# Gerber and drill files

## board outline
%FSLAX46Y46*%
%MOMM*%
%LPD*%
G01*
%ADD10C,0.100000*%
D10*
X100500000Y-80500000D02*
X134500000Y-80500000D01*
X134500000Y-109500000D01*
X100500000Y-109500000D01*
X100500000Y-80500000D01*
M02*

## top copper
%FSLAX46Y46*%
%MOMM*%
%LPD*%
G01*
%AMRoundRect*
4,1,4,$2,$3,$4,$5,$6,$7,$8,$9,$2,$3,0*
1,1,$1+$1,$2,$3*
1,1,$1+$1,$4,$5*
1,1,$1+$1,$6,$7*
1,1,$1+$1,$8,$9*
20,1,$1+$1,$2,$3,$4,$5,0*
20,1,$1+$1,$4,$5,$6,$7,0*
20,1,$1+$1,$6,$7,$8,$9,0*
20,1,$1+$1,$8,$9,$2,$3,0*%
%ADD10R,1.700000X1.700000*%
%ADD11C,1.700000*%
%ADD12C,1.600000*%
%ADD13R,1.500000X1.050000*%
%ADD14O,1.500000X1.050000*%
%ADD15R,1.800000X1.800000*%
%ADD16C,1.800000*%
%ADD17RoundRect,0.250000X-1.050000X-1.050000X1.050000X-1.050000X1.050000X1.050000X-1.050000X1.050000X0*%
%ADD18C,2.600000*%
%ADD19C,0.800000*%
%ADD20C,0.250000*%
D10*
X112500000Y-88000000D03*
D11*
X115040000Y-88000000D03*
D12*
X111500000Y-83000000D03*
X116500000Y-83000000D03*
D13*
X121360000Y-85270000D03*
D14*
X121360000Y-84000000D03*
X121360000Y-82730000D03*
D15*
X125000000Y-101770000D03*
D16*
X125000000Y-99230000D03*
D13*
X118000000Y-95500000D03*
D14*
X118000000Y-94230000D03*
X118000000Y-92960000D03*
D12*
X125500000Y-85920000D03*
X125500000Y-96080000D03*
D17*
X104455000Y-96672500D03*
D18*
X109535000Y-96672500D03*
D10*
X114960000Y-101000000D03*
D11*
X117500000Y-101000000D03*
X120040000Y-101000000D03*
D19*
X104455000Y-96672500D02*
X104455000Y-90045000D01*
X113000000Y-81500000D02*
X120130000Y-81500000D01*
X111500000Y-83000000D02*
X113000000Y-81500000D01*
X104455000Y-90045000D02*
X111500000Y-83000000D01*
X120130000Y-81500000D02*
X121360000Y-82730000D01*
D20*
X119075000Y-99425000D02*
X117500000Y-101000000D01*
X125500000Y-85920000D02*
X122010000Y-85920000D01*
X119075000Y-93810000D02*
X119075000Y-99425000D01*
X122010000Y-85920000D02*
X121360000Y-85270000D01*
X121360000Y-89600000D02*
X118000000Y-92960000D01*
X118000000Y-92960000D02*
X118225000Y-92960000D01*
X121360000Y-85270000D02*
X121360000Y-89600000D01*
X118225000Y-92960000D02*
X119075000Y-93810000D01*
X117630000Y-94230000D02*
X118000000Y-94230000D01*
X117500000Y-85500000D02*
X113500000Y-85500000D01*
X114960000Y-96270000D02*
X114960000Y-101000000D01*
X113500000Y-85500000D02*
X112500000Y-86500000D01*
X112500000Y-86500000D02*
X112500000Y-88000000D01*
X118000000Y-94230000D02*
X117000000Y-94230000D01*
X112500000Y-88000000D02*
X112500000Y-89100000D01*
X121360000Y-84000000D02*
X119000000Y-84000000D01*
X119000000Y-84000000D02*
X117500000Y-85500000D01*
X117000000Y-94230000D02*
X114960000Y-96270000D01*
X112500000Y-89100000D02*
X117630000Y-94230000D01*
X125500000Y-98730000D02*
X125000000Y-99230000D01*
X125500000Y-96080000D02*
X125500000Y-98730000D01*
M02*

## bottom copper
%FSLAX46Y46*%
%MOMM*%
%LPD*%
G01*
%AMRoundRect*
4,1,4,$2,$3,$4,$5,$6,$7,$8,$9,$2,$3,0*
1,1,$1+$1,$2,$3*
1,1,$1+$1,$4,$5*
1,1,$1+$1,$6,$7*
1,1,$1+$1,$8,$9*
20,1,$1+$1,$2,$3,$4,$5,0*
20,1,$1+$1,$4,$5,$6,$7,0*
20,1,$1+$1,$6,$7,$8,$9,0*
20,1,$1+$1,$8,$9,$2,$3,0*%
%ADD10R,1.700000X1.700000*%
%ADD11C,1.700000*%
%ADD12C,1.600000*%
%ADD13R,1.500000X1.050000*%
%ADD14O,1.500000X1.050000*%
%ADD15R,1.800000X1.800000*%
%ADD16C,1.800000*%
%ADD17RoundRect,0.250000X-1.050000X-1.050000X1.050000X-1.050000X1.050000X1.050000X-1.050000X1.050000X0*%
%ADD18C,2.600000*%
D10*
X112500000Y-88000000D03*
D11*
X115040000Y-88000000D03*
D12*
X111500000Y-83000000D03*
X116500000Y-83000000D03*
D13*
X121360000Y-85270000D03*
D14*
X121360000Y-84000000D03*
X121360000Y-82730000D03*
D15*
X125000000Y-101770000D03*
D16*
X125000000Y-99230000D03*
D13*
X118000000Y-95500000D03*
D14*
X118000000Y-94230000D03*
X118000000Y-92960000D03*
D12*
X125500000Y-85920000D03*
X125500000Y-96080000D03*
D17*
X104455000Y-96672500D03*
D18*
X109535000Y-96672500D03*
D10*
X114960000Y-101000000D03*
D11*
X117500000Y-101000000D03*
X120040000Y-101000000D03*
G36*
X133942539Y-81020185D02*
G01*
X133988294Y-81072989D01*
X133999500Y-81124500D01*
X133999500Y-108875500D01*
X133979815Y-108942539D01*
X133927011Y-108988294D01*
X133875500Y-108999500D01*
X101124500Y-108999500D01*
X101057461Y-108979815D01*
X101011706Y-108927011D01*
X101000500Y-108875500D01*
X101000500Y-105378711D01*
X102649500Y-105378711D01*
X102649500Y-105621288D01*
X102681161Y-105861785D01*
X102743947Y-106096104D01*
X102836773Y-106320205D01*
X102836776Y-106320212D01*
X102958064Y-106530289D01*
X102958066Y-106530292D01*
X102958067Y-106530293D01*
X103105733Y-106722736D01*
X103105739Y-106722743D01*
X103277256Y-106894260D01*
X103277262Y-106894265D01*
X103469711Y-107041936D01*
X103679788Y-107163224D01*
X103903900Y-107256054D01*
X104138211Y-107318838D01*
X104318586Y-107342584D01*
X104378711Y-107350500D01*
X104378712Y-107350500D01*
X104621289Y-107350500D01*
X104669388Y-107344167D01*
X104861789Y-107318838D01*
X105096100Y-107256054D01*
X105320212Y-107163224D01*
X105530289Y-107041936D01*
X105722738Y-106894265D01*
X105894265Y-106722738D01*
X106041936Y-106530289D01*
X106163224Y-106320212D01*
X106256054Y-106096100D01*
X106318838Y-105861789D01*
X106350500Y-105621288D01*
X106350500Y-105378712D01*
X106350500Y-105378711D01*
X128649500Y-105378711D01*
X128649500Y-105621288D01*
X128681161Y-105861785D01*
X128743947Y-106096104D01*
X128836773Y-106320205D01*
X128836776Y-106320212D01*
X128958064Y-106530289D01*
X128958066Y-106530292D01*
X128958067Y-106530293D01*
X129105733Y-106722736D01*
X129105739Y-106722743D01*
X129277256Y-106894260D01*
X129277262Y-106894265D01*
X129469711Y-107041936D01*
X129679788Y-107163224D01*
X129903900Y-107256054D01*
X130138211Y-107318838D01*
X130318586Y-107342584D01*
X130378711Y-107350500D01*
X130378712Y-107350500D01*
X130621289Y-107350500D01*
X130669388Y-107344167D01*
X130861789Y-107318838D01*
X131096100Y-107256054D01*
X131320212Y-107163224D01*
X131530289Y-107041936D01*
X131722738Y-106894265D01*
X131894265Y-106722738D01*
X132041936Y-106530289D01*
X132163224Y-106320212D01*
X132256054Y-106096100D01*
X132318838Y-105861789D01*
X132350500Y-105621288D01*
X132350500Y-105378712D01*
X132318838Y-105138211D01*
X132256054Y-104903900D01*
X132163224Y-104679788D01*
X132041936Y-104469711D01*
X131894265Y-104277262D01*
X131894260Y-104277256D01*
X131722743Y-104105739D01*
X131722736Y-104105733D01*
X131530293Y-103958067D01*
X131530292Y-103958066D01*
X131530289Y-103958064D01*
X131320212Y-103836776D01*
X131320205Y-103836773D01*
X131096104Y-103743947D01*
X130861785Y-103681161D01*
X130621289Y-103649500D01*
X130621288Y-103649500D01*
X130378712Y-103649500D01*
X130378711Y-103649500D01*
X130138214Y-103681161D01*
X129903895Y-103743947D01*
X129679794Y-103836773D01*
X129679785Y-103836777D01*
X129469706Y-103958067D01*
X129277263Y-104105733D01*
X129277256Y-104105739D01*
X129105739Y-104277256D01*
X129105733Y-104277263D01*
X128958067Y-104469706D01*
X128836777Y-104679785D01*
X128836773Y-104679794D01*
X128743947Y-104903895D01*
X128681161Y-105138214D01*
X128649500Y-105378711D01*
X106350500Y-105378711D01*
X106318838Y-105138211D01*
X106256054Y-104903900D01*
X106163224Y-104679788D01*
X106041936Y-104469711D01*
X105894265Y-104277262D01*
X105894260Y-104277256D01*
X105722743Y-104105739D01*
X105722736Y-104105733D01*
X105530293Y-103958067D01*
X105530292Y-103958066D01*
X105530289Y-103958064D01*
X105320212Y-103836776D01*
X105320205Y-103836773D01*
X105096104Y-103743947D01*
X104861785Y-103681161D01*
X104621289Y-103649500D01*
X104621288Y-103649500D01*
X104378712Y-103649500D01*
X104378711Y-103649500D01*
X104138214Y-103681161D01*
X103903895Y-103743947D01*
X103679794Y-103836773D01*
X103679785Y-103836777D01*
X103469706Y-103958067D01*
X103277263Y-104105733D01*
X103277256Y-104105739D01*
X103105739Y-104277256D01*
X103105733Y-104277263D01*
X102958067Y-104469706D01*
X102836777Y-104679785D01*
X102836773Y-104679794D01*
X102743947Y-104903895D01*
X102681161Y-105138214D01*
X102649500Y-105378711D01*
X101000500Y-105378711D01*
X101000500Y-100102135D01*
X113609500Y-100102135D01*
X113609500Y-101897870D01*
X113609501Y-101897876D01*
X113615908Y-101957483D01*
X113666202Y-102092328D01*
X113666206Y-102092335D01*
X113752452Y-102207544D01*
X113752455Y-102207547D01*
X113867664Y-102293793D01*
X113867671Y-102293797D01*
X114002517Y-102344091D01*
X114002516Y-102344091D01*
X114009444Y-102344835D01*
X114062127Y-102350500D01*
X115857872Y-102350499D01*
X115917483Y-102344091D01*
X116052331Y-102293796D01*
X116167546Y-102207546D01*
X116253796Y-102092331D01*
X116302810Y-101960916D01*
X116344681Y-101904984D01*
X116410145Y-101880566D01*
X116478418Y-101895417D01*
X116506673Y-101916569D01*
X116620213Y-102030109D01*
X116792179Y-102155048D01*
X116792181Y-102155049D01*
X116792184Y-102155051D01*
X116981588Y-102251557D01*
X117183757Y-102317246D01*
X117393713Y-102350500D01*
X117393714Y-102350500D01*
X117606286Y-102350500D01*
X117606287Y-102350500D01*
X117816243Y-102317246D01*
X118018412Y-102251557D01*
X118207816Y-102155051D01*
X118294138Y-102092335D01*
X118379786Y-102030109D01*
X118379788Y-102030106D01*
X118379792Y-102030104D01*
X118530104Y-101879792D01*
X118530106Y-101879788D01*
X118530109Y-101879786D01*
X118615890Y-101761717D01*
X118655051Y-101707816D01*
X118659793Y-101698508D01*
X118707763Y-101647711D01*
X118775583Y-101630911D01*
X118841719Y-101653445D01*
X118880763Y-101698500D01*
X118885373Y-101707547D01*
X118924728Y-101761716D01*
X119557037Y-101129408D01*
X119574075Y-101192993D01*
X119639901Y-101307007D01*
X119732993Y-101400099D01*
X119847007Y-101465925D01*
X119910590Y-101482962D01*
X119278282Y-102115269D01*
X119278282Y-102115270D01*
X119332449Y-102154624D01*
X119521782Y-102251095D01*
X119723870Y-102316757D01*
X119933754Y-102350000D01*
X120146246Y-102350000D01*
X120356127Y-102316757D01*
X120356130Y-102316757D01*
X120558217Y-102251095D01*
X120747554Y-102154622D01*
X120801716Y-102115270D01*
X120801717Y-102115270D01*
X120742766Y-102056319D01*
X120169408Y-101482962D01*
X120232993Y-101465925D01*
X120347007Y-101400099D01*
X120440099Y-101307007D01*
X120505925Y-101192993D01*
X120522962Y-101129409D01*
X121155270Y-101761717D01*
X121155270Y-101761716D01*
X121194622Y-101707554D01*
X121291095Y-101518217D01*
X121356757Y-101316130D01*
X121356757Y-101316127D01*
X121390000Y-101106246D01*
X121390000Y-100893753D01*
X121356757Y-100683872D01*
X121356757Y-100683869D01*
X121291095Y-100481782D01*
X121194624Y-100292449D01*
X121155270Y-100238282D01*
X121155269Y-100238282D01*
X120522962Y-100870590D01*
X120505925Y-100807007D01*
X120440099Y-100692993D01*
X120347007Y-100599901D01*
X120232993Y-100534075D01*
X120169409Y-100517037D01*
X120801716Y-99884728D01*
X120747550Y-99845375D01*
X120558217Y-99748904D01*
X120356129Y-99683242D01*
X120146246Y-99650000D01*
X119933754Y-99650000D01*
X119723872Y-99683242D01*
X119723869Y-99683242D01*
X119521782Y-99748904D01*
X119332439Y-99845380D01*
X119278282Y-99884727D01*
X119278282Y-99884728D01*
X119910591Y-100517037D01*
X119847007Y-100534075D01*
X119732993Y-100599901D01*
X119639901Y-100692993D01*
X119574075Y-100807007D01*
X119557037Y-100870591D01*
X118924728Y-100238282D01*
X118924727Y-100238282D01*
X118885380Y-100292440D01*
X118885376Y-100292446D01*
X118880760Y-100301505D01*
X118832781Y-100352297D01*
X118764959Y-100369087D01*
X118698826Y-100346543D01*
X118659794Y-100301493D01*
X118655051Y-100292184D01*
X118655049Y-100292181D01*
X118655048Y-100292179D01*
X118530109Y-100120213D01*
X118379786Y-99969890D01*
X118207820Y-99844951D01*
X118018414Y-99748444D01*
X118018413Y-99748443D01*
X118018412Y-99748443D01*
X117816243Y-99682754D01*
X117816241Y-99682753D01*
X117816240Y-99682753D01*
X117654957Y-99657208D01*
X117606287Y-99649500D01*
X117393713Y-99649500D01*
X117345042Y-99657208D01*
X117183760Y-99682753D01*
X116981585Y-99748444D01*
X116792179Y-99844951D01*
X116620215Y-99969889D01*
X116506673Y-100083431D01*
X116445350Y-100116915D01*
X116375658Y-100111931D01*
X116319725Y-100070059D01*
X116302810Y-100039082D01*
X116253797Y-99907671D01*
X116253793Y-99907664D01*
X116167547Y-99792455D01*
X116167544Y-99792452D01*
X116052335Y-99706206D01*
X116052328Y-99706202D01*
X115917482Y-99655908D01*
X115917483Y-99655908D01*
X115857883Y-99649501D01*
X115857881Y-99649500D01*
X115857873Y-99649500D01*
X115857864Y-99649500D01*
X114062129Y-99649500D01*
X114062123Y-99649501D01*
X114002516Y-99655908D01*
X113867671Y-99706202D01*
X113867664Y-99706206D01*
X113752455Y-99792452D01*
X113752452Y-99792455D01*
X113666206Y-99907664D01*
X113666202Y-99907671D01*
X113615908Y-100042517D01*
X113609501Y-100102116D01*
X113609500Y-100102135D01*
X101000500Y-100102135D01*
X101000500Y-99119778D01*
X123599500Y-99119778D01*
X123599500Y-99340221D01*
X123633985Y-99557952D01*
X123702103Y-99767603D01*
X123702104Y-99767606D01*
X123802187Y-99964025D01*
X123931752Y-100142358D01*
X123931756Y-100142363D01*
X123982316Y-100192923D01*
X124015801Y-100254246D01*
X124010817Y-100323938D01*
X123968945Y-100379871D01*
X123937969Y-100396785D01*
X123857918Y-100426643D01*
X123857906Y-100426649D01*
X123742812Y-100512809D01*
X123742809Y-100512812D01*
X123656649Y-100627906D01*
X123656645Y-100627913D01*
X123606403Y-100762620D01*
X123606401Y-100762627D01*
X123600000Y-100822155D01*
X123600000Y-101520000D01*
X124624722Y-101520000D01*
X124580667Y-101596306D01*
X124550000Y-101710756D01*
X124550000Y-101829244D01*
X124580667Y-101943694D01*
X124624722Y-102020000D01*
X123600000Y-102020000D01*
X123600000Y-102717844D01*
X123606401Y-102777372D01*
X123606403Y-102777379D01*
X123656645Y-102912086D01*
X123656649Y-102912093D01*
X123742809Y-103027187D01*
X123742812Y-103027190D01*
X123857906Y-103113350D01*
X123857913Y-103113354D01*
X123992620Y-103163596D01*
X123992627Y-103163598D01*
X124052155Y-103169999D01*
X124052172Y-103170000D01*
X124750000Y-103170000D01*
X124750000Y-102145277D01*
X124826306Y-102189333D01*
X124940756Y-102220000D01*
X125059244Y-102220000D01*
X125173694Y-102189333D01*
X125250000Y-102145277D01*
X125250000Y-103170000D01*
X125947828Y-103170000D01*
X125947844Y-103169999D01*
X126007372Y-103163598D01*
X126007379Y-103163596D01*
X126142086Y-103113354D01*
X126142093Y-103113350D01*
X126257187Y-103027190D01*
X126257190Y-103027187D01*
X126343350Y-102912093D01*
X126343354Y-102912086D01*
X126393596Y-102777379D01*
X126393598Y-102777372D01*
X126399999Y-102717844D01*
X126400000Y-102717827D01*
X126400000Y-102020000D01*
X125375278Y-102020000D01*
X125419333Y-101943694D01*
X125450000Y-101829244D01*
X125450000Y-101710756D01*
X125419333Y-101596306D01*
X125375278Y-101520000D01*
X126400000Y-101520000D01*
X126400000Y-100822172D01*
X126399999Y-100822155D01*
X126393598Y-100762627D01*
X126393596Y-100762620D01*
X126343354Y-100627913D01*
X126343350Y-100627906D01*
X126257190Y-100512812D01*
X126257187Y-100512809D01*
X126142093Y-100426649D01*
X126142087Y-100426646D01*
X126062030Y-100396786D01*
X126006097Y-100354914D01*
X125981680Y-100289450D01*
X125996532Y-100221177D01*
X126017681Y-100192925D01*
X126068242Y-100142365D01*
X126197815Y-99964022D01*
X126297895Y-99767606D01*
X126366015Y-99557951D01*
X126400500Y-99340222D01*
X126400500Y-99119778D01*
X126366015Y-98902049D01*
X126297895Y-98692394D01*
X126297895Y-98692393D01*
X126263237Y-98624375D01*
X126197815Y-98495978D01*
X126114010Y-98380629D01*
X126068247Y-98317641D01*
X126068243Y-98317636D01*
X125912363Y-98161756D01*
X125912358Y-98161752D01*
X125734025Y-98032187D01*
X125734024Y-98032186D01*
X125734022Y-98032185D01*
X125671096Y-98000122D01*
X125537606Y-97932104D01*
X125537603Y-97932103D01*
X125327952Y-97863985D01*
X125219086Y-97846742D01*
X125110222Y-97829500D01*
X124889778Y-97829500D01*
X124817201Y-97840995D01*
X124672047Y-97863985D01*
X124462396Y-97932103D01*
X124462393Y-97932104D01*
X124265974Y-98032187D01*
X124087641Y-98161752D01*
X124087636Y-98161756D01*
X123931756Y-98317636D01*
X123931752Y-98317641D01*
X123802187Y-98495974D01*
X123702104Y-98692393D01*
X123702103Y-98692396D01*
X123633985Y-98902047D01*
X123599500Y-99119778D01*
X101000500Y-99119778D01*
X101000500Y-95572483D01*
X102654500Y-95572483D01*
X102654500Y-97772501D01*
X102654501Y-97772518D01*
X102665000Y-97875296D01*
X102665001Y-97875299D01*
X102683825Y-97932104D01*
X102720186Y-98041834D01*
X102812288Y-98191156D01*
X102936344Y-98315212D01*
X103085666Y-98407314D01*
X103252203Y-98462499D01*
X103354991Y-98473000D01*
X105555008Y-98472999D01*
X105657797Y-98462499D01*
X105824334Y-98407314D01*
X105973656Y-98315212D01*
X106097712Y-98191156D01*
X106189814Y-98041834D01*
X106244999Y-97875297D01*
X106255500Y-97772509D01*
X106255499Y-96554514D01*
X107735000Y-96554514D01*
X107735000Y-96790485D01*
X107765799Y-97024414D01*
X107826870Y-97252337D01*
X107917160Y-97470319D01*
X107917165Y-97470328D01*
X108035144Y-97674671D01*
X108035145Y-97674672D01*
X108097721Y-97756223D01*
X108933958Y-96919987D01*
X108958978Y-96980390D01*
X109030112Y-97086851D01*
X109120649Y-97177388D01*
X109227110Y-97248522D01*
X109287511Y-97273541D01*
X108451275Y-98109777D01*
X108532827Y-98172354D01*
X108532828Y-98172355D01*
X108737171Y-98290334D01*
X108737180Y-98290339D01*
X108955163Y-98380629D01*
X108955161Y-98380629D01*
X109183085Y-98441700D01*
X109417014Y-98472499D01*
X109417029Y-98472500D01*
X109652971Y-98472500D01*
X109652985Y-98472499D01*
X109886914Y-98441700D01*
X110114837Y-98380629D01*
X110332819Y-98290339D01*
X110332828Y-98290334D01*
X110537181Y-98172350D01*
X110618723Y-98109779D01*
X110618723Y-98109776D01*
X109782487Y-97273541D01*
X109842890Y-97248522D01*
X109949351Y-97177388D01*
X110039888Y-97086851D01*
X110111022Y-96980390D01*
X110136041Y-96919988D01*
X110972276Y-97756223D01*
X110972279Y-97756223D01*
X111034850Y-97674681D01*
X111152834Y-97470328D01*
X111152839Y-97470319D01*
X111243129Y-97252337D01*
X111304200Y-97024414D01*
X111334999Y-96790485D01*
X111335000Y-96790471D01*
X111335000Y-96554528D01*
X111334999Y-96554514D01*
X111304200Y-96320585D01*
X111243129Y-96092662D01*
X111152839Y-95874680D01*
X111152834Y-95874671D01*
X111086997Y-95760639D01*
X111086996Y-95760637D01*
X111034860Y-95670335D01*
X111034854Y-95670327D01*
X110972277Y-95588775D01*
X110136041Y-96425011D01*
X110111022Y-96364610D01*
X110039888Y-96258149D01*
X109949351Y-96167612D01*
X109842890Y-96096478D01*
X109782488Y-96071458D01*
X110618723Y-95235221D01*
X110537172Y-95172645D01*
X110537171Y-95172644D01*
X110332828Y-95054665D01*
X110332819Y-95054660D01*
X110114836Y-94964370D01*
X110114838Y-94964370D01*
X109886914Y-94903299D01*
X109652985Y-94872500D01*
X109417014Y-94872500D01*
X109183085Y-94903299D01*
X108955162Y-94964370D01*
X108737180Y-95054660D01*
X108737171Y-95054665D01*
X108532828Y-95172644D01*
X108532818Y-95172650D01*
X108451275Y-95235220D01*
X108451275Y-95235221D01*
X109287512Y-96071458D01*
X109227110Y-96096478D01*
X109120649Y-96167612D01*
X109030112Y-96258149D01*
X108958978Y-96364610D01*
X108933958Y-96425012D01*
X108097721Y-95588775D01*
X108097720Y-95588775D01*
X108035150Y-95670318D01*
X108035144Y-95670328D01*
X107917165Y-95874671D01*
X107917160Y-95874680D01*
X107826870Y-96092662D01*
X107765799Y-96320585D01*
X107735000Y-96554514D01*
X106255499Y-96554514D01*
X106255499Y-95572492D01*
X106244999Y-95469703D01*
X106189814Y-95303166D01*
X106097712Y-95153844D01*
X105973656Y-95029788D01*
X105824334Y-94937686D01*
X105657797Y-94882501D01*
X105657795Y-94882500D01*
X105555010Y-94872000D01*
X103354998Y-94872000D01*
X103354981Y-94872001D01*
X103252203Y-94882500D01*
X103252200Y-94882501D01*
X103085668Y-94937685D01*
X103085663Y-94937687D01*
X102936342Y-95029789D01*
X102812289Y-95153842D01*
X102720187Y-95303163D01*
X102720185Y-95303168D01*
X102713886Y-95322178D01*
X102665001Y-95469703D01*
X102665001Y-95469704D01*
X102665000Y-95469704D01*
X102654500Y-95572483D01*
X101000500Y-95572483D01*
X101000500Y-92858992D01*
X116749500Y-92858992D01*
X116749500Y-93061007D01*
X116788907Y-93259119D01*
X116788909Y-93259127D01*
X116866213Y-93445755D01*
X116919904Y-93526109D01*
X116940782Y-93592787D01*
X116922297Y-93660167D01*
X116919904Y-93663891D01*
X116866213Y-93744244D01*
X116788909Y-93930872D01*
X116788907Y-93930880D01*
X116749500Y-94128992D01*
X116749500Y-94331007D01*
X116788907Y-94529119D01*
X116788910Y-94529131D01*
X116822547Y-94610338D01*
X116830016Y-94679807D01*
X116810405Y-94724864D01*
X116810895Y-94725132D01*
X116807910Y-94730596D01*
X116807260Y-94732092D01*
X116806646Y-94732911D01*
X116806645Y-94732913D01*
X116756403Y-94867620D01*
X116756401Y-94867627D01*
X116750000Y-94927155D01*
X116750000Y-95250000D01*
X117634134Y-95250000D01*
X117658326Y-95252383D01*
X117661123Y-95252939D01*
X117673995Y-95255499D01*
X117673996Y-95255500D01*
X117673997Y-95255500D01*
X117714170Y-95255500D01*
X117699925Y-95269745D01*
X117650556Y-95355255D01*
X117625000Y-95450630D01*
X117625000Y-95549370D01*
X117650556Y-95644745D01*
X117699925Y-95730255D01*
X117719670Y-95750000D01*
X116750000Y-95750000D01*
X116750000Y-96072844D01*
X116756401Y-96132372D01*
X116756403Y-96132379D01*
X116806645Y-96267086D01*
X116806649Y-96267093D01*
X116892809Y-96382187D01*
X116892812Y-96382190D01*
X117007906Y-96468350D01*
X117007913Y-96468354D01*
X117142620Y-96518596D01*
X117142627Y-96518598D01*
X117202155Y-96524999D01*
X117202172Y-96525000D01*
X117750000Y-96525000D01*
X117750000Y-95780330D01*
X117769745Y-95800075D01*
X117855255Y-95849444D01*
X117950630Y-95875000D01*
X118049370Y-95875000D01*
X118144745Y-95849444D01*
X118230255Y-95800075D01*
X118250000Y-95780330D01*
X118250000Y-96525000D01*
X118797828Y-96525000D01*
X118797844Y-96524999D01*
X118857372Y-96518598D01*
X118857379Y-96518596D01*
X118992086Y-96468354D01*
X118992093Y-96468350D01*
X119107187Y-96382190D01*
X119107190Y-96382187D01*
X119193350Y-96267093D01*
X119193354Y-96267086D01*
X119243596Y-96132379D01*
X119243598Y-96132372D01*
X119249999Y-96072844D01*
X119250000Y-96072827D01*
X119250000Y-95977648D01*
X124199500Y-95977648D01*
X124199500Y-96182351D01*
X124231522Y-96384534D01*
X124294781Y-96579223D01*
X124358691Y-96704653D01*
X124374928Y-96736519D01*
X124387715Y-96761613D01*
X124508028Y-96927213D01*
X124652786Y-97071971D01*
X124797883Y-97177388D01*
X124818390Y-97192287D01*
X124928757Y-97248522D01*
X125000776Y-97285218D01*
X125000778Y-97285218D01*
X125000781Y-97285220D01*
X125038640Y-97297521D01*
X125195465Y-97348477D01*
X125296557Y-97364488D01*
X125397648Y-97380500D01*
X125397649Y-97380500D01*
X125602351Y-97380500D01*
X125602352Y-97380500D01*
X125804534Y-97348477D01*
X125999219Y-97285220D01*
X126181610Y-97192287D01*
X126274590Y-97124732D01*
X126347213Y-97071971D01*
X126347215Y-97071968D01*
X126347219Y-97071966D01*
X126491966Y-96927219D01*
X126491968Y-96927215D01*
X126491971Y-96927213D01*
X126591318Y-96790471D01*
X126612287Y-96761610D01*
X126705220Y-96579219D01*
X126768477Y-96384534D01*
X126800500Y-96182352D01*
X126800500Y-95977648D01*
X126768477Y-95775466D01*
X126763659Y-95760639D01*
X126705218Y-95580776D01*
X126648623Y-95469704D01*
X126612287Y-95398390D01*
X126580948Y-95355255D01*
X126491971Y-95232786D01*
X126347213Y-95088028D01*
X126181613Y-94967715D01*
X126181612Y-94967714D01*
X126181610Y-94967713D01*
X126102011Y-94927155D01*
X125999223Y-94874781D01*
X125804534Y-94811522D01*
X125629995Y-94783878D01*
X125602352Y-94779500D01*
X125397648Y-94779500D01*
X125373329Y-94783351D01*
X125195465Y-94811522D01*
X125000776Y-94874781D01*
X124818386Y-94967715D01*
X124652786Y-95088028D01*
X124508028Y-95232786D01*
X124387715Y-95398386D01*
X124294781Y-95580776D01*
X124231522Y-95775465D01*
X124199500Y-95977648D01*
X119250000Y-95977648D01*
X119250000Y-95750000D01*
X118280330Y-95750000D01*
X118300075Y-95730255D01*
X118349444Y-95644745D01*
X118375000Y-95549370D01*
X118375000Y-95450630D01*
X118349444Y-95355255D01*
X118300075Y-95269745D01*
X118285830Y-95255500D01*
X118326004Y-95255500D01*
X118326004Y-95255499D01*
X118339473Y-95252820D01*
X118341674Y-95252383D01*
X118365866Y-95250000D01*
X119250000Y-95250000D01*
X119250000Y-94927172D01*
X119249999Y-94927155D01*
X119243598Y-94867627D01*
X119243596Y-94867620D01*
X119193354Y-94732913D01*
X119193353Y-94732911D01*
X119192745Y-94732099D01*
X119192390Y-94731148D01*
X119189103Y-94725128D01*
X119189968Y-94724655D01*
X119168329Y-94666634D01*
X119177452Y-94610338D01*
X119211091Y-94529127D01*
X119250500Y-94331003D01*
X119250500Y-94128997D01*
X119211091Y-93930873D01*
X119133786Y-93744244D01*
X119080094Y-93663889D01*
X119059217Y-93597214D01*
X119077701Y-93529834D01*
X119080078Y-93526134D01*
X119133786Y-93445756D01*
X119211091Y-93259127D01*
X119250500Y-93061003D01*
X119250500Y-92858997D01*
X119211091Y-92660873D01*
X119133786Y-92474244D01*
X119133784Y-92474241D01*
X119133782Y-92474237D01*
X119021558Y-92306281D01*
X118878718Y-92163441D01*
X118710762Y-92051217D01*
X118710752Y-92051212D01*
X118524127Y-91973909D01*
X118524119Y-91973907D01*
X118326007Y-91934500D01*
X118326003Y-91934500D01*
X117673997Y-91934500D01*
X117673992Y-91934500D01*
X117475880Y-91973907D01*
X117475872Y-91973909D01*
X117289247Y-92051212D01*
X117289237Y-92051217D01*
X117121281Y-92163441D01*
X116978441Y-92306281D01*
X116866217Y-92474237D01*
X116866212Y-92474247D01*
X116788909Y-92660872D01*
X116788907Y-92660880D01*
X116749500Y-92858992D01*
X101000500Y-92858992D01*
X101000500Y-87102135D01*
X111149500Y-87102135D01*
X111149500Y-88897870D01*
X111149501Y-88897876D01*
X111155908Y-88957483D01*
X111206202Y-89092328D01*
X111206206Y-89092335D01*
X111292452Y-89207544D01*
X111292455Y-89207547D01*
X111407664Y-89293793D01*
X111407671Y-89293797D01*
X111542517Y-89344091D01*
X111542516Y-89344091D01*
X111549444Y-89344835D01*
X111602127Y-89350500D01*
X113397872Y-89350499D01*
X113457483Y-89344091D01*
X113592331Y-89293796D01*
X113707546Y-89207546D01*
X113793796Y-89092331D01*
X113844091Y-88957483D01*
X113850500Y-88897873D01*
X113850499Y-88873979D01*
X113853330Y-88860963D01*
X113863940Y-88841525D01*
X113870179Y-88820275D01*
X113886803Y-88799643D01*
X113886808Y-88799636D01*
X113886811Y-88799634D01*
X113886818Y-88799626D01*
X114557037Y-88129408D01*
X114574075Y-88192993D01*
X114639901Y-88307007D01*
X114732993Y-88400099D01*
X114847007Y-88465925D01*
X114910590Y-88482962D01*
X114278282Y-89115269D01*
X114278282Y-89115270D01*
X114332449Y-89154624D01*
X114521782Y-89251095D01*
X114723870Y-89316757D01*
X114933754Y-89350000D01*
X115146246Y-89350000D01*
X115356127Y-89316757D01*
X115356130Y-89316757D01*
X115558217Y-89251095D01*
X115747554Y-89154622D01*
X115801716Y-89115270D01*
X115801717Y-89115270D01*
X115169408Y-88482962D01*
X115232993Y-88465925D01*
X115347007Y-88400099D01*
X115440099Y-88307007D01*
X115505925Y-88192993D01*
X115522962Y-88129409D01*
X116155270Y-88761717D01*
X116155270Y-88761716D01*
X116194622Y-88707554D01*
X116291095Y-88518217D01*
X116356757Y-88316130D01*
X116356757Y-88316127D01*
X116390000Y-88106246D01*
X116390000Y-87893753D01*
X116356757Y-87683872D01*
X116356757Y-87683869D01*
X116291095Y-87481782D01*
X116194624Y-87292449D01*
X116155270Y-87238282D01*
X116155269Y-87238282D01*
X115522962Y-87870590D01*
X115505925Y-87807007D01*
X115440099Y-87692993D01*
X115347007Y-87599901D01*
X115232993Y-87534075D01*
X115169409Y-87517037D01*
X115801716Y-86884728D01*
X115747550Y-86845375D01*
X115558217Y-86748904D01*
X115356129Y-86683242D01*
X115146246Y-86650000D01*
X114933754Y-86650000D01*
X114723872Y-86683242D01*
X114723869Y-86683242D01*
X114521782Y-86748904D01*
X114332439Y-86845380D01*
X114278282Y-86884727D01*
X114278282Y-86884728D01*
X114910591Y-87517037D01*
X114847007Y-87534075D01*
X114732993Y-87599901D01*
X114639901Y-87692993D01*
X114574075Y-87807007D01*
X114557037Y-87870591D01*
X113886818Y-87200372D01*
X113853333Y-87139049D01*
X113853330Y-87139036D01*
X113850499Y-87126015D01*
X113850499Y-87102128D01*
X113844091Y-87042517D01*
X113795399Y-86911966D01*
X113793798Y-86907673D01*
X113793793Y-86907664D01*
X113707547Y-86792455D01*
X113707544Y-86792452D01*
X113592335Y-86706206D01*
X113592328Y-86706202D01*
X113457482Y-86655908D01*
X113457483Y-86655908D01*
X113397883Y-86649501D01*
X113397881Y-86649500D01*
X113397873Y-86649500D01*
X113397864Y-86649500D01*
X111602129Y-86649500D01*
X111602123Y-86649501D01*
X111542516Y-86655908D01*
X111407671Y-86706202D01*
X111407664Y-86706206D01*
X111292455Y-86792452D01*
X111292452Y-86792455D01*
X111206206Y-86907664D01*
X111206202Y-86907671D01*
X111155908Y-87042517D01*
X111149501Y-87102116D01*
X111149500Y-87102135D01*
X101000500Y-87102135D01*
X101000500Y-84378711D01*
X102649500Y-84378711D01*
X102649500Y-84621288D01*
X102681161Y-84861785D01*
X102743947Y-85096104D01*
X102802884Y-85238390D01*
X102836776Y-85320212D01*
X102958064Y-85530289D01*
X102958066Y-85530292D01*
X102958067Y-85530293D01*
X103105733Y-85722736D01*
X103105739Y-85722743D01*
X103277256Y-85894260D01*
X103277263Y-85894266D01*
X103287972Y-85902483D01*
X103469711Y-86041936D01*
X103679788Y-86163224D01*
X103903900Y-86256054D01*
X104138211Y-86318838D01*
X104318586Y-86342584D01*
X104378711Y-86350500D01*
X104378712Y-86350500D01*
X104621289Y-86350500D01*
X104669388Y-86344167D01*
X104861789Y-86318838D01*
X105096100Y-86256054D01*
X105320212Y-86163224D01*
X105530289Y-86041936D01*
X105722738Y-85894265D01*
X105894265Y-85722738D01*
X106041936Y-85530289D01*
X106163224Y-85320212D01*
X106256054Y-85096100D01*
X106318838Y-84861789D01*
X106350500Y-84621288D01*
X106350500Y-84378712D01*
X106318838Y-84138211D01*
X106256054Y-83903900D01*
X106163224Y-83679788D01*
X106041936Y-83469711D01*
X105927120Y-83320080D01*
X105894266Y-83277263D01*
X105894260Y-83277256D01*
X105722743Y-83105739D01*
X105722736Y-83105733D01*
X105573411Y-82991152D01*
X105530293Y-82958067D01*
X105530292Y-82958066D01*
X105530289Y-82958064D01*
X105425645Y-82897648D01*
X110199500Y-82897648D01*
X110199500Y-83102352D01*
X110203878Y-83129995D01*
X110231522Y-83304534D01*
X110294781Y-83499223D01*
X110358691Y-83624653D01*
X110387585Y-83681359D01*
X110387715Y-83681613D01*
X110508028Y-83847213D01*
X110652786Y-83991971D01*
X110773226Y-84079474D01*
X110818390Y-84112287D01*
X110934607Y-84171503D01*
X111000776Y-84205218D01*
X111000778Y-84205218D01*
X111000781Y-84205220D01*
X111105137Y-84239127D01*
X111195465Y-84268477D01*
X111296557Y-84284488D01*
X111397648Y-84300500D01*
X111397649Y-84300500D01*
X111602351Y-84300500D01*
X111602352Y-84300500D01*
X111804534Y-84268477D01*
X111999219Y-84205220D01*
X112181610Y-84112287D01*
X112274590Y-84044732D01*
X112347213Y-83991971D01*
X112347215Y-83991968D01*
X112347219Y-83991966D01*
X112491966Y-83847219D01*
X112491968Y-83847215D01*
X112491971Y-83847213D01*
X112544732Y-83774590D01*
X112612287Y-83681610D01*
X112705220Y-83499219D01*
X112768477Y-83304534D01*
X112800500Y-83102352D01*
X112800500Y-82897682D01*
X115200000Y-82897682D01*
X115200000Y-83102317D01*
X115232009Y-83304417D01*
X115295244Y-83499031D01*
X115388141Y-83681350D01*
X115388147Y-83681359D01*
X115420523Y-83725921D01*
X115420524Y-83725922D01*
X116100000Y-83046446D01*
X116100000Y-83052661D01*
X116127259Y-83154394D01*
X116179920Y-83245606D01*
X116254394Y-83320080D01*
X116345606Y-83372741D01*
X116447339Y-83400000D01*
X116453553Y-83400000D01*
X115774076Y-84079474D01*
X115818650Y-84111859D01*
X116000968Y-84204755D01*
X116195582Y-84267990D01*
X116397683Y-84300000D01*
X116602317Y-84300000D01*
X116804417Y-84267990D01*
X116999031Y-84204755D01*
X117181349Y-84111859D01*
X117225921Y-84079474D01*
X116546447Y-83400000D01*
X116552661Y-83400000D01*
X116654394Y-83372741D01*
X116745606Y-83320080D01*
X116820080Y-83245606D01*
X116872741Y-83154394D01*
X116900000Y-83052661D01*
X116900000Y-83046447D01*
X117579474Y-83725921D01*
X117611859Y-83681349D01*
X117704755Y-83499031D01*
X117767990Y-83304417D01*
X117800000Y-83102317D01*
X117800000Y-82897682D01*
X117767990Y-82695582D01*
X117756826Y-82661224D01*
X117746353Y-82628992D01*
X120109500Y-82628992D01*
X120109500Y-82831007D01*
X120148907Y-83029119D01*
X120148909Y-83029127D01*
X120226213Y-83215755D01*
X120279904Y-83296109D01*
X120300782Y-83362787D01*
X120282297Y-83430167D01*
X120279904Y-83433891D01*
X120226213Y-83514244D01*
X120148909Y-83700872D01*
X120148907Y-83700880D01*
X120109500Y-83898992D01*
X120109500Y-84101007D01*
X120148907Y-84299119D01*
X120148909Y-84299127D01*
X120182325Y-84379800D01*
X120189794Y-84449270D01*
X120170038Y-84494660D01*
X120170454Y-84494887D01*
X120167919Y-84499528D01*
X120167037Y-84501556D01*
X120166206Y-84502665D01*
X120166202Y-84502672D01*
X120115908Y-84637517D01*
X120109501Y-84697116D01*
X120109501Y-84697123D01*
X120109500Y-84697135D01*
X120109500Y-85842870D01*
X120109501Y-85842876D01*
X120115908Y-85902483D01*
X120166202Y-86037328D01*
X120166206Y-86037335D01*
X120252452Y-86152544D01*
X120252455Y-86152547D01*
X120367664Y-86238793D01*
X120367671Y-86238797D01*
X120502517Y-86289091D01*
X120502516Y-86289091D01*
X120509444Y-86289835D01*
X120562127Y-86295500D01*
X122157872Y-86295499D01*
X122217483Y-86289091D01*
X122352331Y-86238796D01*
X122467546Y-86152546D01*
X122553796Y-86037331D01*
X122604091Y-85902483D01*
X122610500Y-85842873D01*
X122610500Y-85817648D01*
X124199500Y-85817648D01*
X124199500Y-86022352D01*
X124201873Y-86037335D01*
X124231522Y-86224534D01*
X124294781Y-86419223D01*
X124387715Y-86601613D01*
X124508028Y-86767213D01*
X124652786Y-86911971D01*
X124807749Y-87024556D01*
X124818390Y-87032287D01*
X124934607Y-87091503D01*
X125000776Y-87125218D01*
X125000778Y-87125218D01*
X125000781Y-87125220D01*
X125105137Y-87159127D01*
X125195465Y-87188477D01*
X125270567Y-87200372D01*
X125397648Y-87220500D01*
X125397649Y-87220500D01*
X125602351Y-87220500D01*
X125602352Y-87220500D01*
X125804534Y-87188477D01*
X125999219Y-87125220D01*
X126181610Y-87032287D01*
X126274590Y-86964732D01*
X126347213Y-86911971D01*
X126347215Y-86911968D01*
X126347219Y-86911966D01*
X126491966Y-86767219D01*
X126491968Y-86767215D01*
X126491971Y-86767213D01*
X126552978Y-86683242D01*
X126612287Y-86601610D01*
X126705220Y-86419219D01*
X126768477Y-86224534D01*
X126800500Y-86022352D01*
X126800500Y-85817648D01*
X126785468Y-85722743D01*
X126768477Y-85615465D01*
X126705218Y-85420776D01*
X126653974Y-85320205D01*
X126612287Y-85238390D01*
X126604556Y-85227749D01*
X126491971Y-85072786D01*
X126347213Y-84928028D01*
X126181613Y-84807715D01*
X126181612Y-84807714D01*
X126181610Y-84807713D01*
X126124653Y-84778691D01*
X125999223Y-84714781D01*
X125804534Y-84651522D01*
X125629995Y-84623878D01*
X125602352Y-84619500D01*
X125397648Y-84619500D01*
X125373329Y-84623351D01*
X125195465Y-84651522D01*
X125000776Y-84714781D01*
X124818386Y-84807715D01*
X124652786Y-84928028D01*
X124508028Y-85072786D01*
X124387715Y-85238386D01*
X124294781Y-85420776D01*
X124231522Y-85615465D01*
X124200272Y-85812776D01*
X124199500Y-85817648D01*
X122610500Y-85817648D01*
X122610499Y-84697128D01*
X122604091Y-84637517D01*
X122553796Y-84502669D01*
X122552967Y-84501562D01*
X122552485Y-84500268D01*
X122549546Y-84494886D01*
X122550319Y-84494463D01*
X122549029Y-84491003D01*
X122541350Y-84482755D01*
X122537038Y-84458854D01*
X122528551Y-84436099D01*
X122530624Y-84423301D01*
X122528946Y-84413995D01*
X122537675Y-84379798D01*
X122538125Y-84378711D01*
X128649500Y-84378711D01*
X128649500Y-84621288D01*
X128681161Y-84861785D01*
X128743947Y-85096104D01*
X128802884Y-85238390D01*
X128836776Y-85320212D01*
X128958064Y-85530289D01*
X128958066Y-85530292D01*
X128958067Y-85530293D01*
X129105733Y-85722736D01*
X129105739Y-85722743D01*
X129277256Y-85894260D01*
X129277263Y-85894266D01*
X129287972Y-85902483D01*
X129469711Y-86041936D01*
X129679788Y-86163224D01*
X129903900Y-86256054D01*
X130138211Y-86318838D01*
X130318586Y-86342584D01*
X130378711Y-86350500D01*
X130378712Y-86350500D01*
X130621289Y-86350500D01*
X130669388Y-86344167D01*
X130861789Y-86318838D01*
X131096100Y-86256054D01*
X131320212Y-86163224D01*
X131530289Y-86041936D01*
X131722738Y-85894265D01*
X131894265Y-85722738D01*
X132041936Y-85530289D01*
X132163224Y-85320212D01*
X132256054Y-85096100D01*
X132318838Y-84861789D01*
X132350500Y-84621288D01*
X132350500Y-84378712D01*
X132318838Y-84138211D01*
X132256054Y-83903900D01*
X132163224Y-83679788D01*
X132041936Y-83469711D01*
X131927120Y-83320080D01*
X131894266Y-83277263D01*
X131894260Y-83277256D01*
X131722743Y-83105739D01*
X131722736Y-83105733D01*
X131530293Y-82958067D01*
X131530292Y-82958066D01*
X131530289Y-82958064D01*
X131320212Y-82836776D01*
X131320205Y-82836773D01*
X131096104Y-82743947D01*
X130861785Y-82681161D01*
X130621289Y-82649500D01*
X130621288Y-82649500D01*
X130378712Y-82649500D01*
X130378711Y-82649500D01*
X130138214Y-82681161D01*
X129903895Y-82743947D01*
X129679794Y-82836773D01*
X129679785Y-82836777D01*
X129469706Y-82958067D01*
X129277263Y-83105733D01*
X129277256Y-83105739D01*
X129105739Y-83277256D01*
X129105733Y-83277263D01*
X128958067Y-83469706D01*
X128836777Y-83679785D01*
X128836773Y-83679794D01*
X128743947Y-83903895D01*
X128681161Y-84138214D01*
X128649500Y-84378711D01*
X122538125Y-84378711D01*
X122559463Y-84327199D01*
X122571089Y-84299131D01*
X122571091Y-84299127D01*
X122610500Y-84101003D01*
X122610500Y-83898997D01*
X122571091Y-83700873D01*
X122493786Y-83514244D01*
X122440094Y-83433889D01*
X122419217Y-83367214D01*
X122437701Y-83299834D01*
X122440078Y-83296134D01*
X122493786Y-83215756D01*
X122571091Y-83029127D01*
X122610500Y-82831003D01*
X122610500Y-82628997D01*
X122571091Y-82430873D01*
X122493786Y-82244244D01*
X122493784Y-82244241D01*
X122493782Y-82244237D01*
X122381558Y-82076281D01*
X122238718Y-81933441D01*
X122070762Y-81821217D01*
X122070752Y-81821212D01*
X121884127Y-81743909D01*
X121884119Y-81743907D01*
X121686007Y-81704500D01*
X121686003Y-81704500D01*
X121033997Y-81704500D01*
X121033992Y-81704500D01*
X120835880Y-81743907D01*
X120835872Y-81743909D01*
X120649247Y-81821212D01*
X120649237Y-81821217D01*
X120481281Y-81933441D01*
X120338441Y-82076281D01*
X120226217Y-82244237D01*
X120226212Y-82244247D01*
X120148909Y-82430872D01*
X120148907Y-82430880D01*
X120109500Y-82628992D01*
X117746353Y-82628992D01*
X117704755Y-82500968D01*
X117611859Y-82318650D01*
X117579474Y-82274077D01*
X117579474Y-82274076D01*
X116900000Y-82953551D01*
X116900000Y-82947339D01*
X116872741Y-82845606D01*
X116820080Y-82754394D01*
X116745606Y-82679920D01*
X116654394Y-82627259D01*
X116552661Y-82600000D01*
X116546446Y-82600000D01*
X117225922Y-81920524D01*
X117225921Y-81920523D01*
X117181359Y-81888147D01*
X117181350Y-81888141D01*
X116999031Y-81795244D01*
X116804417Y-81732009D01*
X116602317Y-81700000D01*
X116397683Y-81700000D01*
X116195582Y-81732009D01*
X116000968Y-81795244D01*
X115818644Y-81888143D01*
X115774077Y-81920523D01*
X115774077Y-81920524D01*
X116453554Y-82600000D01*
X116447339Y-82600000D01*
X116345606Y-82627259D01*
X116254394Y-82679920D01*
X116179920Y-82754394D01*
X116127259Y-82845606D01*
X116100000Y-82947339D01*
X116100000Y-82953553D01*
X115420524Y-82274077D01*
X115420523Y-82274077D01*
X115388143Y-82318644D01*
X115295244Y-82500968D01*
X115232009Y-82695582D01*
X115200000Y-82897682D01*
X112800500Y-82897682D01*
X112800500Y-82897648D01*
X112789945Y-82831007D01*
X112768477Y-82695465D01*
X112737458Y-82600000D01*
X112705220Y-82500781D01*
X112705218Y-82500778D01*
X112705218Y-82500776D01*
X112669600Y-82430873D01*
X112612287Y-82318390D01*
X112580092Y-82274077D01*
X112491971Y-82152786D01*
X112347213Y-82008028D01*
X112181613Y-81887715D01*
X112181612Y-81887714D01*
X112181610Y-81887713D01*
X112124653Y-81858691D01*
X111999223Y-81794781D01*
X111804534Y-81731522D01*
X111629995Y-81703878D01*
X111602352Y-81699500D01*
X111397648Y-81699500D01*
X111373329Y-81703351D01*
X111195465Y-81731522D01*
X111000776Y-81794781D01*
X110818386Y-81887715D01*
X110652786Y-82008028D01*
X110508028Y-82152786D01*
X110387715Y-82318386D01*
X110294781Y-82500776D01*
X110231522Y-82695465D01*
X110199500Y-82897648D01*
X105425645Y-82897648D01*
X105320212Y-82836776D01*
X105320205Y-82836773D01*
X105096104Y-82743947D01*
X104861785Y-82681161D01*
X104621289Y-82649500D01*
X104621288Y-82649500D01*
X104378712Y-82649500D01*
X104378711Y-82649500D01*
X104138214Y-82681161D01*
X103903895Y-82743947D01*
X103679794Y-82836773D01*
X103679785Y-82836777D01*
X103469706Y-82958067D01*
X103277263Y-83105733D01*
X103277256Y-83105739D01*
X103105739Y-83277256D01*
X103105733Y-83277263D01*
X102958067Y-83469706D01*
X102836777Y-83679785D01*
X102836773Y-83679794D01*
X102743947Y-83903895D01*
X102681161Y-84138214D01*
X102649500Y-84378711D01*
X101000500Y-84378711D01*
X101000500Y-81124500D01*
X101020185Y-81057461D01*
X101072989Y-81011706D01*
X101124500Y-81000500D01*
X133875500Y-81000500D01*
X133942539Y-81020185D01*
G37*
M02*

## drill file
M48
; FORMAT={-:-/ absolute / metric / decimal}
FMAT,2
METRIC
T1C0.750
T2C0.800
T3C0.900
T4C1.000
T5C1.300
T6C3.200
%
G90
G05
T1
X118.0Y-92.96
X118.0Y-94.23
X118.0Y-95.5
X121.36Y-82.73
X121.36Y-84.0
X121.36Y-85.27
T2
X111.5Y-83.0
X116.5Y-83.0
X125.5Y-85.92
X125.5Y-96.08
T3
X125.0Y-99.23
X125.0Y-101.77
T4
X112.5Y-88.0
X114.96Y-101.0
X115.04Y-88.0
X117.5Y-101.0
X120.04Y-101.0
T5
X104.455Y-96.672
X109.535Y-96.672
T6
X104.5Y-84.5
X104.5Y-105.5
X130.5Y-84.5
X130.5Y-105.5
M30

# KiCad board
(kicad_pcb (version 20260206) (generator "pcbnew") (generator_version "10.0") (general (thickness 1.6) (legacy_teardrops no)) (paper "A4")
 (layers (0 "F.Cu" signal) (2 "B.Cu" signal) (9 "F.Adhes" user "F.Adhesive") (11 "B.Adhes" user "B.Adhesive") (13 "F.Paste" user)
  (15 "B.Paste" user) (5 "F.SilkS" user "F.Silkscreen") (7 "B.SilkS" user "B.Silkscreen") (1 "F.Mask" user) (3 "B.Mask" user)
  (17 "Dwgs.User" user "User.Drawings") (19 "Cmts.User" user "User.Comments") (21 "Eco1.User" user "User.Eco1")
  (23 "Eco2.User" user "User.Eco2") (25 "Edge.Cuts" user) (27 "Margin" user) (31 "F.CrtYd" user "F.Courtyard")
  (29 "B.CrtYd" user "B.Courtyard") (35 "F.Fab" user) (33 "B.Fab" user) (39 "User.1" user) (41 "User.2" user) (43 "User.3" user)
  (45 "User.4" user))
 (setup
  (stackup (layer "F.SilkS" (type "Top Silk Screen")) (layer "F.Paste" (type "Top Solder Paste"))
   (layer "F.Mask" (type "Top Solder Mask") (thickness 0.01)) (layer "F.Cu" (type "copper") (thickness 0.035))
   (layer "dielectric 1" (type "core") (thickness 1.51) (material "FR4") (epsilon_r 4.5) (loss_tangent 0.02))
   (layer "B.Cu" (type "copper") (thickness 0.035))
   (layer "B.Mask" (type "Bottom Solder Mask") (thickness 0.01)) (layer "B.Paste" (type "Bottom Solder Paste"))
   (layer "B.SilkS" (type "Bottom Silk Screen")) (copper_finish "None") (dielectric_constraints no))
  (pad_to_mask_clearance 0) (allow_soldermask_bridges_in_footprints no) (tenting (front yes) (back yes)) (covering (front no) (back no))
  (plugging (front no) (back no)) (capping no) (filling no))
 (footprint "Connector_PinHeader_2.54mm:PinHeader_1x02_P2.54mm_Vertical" (layer "F.Cu") (at 112.5 88 90)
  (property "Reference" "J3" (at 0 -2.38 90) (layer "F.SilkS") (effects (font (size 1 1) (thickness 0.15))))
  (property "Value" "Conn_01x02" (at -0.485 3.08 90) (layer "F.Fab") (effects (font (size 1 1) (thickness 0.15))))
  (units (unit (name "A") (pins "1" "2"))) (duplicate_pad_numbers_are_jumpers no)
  (pad "1" thru_hole rect (at 0 0 90) (size 1.7 1.7) (drill 1) (layers "*.Cu" "*.Mask") (remove_unused_layers no) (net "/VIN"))
  (pad "2" thru_hole circle (at 0 2.54 90) (size 1.7 1.7) (drill 1) (layers "*.Cu" "*.Mask") (remove_unused_layers no) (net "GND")))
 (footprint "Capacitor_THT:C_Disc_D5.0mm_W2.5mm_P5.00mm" (layer "F.Cu") (at 111.5 83)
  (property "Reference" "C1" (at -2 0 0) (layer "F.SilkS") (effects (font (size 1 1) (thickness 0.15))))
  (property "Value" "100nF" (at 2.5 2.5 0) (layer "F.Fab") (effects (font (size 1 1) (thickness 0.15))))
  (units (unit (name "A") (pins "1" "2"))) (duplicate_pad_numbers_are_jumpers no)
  (pad "1" thru_hole circle (at 0 0) (size 1.6 1.6) (drill 0.8) (layers "*.Cu" "*.Mask") (remove_unused_layers no) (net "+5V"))
  (pad "2" thru_hole circle (at 5 0) (size 1.6 1.6) (drill 0.8) (layers "*.Cu" "*.Mask") (remove_unused_layers no) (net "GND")))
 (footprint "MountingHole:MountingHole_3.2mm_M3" (layer "F.Cu") (at 104.5 84.5)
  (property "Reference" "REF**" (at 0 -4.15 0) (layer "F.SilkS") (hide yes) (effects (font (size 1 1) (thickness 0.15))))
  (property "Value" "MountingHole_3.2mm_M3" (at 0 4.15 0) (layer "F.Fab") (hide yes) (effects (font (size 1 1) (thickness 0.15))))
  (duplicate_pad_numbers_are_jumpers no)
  (pad "" np_thru_hole circle (at 0 0) (size 3.2 3.2) (drill 3.2) (layers "*.Cu" "*.Mask")))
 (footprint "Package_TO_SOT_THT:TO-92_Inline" (layer "F.Cu") (at 121.36 85.27 90)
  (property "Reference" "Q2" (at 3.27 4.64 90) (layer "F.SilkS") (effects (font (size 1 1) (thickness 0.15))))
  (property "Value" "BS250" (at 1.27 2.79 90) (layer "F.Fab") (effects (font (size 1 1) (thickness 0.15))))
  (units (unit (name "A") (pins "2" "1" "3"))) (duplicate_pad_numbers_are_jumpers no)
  (pad "1" thru_hole rect (at 0 0 90) (size 1.05 1.5) (drill 0.75) (layers "*.Cu" "*.Mask") (remove_unused_layers no) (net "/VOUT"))
  (pad "2" thru_hole oval (at 1.27 0 90) (size 1.05 1.5) (drill 0.75) (layers "*.Cu" "*.Mask") (remove_unused_layers no) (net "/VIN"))
  (pad "3" thru_hole oval (at 2.54 0 90) (size 1.05 1.5) (drill 0.75) (layers "*.Cu" "*.Mask") (remove_unused_layers no) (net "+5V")))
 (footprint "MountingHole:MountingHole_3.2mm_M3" (layer "F.Cu") (at 130.5 84.5)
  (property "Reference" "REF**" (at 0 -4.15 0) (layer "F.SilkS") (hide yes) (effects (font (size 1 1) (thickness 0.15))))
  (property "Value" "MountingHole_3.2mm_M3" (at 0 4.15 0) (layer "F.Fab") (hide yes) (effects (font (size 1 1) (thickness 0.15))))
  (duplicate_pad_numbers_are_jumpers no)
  (pad "" np_thru_hole circle (at 0 0) (size 3.2 3.2) (drill 3.2) (layers "*.Cu" "*.Mask")))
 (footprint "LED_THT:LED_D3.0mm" (layer "F.Cu") (at 125 101.77 90)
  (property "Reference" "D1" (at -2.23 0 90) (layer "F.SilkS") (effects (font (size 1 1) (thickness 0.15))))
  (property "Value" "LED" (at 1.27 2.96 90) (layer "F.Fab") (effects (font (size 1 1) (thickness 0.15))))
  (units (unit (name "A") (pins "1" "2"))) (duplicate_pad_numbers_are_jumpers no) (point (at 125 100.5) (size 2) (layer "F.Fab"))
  (pad "1" thru_hole rect (at 0 0 90) (size 1.8 1.8) (drill 0.9) (layers "*.Cu" "*.Mask") (remove_unused_layers no) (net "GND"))
  (pad "2" thru_hole circle (at 2.54 0 90) (size 1.8 1.8) (drill 0.9) (layers "*.Cu" "*.Mask") (remove_unused_layers no) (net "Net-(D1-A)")))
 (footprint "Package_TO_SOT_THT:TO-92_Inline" (layer "F.Cu") (at 118 95.5 90)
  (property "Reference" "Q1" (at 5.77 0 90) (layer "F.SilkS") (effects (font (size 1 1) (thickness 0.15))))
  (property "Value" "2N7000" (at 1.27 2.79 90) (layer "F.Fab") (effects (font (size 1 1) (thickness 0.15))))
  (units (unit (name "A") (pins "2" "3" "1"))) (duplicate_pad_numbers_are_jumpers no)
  (pad "1" thru_hole rect (at 0 0 90) (size 1.05 1.5) (drill 0.75) (layers "*.Cu" "*.Mask") (remove_unused_layers no) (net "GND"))
  (pad "2" thru_hole oval (at 1.27 0 90) (size 1.05 1.5) (drill 0.75) (layers "*.Cu" "*.Mask") (remove_unused_layers no) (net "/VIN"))
  (pad "3" thru_hole oval (at 2.54 0 90) (size 1.05 1.5) (drill 0.75) (layers "*.Cu" "*.Mask") (remove_unused_layers no) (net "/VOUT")))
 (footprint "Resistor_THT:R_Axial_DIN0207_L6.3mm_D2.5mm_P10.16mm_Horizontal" (layer "F.Cu") (at 125.5 85.92 -90)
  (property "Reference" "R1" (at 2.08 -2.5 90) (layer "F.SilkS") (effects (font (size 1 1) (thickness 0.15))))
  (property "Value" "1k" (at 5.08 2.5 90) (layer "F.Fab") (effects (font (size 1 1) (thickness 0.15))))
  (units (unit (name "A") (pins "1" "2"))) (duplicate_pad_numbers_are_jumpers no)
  (pad "1" thru_hole circle (at 0 0 270) (size 1.6 1.6) (drill 0.8) (layers "*.Cu" "*.Mask") (remove_unused_layers no) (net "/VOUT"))
  (pad "2" thru_hole circle (at 10.16 0 270) (size 1.6 1.6) (drill 0.8) (layers "*.Cu" "*.Mask") (remove_unused_layers no)
   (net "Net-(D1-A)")))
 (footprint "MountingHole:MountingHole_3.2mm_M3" (layer "F.Cu") (at 104.5 105.5)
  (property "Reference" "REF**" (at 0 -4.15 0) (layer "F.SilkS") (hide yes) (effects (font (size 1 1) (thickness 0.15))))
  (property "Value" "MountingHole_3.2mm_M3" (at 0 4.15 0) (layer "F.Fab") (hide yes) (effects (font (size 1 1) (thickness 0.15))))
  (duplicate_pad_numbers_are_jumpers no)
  (pad "" np_thru_hole circle (at 0 0) (size 3.2 3.2) (drill 3.2) (layers "*.Cu" "*.Mask")))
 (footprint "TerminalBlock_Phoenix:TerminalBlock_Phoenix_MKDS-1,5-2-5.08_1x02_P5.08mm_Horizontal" (layer "F.Cu") (at 104.455 96.6725)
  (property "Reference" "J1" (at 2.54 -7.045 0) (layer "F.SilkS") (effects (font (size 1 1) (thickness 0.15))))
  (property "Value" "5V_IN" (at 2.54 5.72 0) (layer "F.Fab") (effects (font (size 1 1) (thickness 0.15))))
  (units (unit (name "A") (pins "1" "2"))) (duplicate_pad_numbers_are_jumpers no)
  (pad "1" thru_hole roundrect (at 0 0) (size 2.6 2.6) (drill 1.3) (layers "*.Cu" "*.Mask") (remove_unused_layers no)
   (roundrect_rratio 0.096154) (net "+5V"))
  (pad "2" thru_hole circle (at 5.08 0) (size 2.6 2.6) (drill 1.3) (layers "*.Cu" "*.Mask") (remove_unused_layers no) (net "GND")))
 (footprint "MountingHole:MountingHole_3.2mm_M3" (layer "F.Cu") (at 130.5 105.5)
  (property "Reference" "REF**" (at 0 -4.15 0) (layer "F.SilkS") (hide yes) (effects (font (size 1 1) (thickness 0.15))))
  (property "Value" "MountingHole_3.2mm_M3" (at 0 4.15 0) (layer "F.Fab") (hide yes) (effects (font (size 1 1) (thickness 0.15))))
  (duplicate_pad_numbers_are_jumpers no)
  (pad "" np_thru_hole circle (at 0 0) (size 3.2 3.2) (drill 3.2) (layers "*.Cu" "*.Mask")))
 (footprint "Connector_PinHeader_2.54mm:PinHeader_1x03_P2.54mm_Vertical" (layer "F.Cu") (at 114.96 101 90)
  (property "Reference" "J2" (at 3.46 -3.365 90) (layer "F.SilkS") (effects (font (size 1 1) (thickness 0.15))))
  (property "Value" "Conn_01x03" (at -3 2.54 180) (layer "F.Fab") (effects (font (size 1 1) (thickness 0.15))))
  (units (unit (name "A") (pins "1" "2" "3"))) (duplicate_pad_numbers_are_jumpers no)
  (pad "1" thru_hole rect (at 0 0 90) (size 1.7 1.7) (drill 1) (layers "*.Cu" "*.Mask") (remove_unused_layers no) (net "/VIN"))
  (pad "2" thru_hole circle (at 0 2.54 90) (size 1.7 1.7) (drill 1) (layers "*.Cu" "*.Mask") (remove_unused_layers no) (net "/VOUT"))
  (pad "3" thru_hole circle (at 0 5.08 90) (size 1.7 1.7) (drill 1) (layers "*.Cu" "*.Mask") (remove_unused_layers no) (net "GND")))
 (gr_rect (start 100.5 80.5) (end 134.5 109.5) (stroke (width 0.1) (type solid)) (fill no) (layer "Edge.Cuts"))
 (segment (start 104.455 96.6725) (end 104.455 90.045) (width 0.8) (layer "F.Cu") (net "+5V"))
 (segment (start 113 81.5) (end 120.13 81.5) (width 0.8) (layer "F.Cu") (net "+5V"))
 (segment (start 111.5 83) (end 113 81.5) (width 0.8) (layer "F.Cu") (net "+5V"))
 (segment (start 104.455 90.045) (end 111.5 83) (width 0.8) (layer "F.Cu") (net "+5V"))
 (segment (start 120.13 81.5) (end 121.36 82.73) (width 0.8) (layer "F.Cu") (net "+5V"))
 (segment (start 119.075 99.425) (end 117.5 101) (width 0.25) (layer "F.Cu") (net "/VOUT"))
 (segment (start 125.5 85.92) (end 122.01 85.92) (width 0.25) (layer "F.Cu") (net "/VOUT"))
 (segment (start 119.075 93.81) (end 119.075 99.425) (width 0.25) (layer "F.Cu") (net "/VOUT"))
 (segment (start 122.01 85.92) (end 121.36 85.27) (width 0.25) (layer "F.Cu") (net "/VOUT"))
 (segment (start 121.36 89.6) (end 118 92.96) (width 0.25) (layer "F.Cu") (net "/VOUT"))
 (segment (start 118 92.96) (end 118.225 92.96) (width 0.25) (layer "F.Cu") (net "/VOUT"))
 (segment (start 121.36 85.27) (end 121.36 89.6) (width 0.25) (layer "F.Cu") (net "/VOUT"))
 (segment (start 118.225 92.96) (end 119.075 93.81) (width 0.25) (layer "F.Cu") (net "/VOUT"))
 (segment (start 117.63 94.23) (end 118 94.23) (width 0.25) (layer "F.Cu") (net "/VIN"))
 (segment (start 117.5 85.5) (end 113.5 85.5) (width 0.25) (layer "F.Cu") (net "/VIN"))
 (segment (start 114.96 96.27) (end 114.96 101) (width 0.25) (layer "F.Cu") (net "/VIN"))
 (segment (start 113.5 85.5) (end 112.5 86.5) (width 0.25) (layer "F.Cu") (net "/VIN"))
 (segment (start 112.5 86.5) (end 112.5 88) (width 0.25) (layer "F.Cu") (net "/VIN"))
 (segment (start 118 94.23) (end 117 94.23) (width 0.25) (layer "F.Cu") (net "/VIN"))
 (segment (start 112.5 88) (end 112.5 89.1) (width 0.25) (layer "F.Cu") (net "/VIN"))
 (segment (start 121.36 84) (end 119 84) (width 0.25) (layer "F.Cu") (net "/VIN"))
 (segment (start 119 84) (end 117.5 85.5) (width 0.25) (layer "F.Cu") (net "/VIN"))
 (segment (start 117 94.23) (end 114.96 96.27) (width 0.25) (layer "F.Cu") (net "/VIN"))
 (segment (start 112.5 89.1) (end 117.63 94.23) (width 0.25) (layer "F.Cu") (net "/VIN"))
 (segment (start 125.5 98.73) (end 125 99.23) (width 0.25) (layer "F.Cu") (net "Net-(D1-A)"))
 (segment (start 125.5 96.08) (end 125.5 98.73) (width 0.25) (layer "F.Cu") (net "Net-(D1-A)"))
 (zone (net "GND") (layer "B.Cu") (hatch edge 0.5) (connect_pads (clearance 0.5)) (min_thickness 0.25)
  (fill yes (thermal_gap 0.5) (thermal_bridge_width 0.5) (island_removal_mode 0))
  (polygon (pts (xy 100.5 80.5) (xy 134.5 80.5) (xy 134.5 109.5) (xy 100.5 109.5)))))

